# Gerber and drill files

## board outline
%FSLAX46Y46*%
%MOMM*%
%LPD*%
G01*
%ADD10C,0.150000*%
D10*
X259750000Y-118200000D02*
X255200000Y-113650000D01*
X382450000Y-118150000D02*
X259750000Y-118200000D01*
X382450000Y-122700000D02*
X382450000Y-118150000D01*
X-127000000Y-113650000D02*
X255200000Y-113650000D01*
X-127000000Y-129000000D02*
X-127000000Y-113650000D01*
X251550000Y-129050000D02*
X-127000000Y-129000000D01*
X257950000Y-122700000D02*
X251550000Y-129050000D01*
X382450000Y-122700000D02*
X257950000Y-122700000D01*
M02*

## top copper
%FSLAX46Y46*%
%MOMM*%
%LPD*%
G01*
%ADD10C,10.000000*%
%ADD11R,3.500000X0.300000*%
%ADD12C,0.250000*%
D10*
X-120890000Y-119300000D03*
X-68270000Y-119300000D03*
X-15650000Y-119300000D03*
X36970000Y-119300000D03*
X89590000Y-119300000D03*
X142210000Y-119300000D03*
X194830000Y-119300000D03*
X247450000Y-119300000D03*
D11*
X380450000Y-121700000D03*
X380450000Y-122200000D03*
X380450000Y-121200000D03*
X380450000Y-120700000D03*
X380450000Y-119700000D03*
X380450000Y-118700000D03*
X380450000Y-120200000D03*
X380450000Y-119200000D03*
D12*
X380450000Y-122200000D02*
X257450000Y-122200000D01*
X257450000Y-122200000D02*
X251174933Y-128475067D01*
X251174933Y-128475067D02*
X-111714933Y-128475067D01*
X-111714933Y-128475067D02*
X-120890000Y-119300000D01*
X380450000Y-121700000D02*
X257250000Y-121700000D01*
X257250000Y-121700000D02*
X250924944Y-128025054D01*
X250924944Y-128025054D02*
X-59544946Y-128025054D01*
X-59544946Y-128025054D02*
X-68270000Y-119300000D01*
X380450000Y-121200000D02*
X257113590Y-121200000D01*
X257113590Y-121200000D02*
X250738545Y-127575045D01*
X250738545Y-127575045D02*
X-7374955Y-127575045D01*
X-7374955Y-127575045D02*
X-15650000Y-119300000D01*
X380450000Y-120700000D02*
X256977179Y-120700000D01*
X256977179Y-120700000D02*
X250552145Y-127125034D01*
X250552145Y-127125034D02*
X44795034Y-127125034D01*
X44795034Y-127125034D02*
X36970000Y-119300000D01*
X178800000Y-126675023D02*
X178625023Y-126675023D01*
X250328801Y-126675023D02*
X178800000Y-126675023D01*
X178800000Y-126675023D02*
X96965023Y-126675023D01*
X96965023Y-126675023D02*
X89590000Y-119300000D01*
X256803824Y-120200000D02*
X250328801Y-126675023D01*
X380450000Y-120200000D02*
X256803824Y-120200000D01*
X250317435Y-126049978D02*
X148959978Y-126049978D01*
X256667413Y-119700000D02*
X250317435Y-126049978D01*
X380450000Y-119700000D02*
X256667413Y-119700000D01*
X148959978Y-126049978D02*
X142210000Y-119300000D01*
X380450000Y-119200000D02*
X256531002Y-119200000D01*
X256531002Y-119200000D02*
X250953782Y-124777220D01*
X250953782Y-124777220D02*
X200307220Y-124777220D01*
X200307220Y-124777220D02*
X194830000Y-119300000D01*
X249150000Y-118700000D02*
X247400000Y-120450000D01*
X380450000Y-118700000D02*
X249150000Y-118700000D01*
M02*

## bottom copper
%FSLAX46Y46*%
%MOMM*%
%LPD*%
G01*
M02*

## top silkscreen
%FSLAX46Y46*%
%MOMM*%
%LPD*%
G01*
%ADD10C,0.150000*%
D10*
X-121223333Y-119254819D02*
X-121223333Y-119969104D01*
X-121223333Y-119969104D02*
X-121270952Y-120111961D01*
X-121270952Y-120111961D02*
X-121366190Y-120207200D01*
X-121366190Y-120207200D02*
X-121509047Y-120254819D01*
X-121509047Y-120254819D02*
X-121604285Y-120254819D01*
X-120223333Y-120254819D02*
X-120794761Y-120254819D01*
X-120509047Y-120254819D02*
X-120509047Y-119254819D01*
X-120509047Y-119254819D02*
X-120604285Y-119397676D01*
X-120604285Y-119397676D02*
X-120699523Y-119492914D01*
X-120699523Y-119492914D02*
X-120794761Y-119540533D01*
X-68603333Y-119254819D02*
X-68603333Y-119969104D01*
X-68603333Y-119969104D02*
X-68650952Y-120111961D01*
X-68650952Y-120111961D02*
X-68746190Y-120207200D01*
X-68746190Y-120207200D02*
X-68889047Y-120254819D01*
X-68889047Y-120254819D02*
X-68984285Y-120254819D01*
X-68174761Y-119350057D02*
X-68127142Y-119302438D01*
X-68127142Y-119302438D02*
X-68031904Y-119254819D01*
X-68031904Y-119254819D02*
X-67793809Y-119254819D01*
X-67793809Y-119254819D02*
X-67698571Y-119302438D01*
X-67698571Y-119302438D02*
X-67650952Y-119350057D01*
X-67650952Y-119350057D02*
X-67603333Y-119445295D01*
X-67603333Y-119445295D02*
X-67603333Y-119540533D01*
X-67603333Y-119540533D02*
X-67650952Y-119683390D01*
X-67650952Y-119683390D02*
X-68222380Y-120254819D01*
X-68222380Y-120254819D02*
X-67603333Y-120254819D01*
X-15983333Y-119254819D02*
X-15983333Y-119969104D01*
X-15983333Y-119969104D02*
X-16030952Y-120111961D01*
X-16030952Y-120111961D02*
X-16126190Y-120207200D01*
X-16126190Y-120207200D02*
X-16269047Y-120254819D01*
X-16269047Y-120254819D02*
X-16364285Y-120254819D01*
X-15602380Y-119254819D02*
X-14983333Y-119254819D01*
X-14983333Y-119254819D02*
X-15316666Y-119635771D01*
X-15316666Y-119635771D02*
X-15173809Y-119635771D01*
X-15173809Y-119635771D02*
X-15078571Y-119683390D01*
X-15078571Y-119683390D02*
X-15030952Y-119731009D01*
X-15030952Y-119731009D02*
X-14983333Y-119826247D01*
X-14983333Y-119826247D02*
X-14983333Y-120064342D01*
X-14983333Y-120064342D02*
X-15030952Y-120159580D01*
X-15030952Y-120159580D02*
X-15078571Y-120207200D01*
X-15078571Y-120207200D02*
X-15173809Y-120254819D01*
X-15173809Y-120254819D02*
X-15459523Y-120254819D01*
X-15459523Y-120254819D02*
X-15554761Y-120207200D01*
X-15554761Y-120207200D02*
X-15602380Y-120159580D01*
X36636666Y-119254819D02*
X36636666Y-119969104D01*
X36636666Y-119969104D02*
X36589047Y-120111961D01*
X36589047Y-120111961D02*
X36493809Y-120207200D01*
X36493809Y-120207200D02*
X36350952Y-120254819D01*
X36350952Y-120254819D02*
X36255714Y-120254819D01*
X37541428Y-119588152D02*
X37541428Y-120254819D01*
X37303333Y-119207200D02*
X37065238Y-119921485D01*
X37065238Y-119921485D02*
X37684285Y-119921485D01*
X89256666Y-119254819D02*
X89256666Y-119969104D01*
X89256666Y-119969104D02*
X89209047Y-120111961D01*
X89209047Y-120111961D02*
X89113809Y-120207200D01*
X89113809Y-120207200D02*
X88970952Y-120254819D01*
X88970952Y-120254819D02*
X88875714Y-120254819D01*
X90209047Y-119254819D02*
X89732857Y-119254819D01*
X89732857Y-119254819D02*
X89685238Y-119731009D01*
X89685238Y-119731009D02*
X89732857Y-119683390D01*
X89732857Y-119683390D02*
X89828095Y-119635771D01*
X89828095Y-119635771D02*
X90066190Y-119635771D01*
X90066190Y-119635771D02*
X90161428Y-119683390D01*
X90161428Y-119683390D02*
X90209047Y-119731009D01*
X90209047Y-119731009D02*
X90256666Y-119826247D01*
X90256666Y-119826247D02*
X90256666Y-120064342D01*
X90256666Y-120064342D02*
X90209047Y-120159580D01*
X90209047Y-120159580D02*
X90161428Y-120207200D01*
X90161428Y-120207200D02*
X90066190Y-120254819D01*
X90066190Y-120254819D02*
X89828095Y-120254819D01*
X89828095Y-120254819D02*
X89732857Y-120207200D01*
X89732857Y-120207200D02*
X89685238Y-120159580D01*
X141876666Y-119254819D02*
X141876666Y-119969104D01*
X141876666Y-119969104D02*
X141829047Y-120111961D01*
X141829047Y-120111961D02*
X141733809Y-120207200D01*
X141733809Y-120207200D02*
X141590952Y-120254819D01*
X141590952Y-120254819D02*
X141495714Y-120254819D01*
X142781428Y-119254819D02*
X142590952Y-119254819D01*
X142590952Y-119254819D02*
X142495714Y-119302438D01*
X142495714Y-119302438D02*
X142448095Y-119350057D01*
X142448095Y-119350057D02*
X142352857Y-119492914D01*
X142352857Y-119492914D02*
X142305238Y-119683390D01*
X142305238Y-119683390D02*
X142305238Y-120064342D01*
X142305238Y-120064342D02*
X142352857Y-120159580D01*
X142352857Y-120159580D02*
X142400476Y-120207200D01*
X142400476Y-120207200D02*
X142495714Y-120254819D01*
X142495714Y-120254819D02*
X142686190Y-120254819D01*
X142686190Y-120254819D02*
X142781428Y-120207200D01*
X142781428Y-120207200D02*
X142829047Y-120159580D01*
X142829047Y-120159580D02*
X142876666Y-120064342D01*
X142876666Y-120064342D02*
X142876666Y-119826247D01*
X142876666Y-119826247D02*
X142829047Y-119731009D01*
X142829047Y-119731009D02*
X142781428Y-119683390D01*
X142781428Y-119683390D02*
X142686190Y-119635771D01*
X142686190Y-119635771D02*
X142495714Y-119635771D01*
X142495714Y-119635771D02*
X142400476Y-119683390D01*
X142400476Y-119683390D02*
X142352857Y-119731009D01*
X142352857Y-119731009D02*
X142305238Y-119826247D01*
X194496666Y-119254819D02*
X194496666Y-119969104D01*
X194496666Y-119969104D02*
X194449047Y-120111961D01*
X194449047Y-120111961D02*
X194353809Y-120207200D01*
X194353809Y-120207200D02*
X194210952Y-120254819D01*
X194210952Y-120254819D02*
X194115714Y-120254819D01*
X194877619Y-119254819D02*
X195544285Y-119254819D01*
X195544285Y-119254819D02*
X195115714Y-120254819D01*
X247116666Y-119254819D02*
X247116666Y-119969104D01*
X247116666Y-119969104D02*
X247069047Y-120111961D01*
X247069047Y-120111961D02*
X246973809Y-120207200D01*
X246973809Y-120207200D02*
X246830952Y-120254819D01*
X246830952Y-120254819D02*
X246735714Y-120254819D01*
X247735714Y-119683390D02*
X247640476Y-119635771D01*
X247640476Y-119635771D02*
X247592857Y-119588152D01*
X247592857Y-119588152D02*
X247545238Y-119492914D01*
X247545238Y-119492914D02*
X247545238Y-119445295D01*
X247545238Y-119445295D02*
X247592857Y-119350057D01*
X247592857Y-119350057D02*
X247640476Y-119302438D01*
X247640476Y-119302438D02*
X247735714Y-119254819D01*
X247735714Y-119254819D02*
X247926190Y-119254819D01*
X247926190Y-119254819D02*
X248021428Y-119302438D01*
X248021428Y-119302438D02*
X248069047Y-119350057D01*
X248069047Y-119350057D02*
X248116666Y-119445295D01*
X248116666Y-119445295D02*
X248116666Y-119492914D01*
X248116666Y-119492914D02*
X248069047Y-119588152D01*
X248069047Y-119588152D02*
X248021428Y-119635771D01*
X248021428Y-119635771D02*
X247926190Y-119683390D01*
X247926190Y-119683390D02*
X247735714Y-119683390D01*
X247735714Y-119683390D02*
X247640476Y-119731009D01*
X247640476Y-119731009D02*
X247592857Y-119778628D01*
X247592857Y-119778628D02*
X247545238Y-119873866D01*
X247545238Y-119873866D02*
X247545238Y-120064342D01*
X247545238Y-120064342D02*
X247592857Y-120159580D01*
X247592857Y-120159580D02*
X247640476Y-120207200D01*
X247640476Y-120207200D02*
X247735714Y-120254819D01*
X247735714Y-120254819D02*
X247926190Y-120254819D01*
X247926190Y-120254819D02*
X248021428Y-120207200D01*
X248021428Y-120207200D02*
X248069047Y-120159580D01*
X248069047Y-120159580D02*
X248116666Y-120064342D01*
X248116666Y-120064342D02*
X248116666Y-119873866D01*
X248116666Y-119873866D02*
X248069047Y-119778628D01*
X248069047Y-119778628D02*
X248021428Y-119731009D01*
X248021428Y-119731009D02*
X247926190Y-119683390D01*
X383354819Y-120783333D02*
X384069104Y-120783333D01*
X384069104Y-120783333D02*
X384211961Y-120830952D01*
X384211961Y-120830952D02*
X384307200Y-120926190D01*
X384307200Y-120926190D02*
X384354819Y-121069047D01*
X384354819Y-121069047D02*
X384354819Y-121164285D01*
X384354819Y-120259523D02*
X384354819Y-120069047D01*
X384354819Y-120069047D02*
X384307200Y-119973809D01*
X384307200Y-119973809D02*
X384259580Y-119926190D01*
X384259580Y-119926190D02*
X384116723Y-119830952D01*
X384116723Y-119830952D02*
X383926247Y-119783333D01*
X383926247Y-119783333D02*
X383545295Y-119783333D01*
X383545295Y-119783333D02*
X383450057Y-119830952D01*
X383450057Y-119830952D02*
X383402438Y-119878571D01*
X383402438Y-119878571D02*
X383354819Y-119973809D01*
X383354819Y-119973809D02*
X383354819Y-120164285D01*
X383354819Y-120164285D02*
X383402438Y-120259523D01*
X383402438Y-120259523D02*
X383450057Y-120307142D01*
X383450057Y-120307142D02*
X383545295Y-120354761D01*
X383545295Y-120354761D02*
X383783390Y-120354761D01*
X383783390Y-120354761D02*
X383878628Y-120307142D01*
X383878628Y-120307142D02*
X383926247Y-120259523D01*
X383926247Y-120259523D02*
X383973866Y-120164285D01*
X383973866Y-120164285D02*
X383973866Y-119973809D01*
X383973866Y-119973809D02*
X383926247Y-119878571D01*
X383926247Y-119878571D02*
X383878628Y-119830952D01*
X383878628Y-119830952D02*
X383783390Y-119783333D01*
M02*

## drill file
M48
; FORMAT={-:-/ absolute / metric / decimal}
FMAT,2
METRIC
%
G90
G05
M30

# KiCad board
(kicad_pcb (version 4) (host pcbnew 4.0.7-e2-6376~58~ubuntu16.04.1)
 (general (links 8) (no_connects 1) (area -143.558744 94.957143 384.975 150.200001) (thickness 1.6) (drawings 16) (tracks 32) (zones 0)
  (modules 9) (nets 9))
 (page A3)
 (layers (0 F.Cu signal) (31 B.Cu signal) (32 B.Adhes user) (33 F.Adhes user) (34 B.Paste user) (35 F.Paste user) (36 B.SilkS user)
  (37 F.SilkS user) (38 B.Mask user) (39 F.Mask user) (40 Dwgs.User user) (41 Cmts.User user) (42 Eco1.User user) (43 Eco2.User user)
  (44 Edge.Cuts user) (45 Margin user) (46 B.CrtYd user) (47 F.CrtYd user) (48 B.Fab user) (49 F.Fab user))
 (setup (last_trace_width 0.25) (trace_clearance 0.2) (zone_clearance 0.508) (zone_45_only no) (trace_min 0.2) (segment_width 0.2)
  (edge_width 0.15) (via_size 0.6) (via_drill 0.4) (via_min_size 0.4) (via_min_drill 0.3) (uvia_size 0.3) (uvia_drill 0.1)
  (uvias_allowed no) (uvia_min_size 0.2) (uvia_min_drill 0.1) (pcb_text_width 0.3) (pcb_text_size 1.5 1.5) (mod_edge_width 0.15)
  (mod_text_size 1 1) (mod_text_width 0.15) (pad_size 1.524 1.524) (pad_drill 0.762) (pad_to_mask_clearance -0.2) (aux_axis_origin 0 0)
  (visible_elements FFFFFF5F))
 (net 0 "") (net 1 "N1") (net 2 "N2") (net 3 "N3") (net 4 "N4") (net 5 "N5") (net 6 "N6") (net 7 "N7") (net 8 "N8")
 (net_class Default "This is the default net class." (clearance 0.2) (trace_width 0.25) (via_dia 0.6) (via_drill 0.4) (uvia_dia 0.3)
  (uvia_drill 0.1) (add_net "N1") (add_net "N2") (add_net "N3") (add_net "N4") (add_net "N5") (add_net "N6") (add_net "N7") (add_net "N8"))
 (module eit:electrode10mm (layer F.Cu) (at -120.89 119.3)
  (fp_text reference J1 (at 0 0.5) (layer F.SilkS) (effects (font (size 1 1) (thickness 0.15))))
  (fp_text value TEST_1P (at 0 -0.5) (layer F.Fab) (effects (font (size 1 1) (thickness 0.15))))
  (pad 1 smd circle (at 0 0) (size 10 10) (layers F.Cu F.Mask) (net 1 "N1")))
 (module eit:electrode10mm (layer F.Cu) (at -68.27 119.3)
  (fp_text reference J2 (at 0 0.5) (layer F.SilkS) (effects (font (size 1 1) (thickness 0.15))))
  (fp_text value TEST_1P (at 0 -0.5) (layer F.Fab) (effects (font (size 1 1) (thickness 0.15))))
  (pad 1 smd circle (at 0 0) (size 10 10) (layers F.Cu F.Mask) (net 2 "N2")))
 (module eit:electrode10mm (layer F.Cu) (at -15.65 119.3)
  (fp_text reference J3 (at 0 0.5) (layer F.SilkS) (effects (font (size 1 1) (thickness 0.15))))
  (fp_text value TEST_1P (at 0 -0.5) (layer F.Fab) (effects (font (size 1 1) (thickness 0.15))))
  (pad 1 smd circle (at 0 0) (size 10 10) (layers F.Cu F.Mask) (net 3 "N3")))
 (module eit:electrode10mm (layer F.Cu) (at 36.97 119.3)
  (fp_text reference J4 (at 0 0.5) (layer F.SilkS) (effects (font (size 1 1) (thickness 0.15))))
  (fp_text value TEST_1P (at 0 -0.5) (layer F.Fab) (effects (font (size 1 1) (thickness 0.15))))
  (pad 1 smd circle (at 0 0) (size 10 10) (layers F.Cu F.Mask) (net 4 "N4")))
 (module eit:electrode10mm (layer F.Cu) (at 89.59 119.3)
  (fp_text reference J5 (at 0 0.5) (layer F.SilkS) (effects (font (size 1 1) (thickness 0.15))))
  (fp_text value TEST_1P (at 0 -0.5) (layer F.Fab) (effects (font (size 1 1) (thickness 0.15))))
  (pad 1 smd circle (at 0 0) (size 10 10) (layers F.Cu F.Mask) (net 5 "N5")))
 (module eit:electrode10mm (layer F.Cu) (at 142.21 119.3)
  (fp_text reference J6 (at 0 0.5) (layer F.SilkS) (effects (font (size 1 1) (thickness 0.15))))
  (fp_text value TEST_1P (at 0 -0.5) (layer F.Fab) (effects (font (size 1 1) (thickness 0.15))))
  (pad 1 smd circle (at 0 0) (size 10 10) (layers F.Cu F.Mask) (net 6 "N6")))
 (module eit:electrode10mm (layer F.Cu) (at 194.83 119.3)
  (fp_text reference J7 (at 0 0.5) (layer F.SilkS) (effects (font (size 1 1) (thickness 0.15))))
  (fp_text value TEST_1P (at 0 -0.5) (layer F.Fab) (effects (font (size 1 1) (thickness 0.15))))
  (pad 1 smd circle (at 0 0) (size 10 10) (layers F.Cu F.Mask) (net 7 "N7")))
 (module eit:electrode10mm (layer F.Cu) (at 247.45 119.3)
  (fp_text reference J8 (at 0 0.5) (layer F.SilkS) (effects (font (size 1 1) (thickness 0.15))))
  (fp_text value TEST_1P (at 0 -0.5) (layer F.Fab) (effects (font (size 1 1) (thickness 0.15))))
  (pad 1 smd circle (at 0 0) (size 10 10) (layers F.Cu F.Mask) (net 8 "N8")))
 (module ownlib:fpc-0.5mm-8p (layer F.Cu) (at 383.4 120.45 90)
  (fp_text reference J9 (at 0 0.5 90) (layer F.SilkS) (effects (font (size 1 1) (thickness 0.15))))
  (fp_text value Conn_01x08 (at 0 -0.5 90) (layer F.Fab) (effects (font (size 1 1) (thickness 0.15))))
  (pad 2 smd rect (at -1.25 -2.95 90) (size 0.3 3.5) (layers F.Cu F.Paste F.Mask) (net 2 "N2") (solder_mask_margin 0.2))
  (pad 1 smd rect (at -1.75 -2.95 90) (size 0.3 3.5) (layers F.Cu F.Paste F.Mask) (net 1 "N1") (solder_mask_margin 0.2))
  (pad 3 smd rect (at -0.75 -2.95 90) (size 0.3 3.5) (layers F.Cu F.Paste F.Mask) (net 3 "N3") (solder_mask_margin 0.2))
  (pad 4 smd rect (at -0.25 -2.95 90) (size 0.3 3.5) (layers F.Cu F.Paste F.Mask) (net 4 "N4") (solder_mask_margin 0.2))
  (pad 6 smd rect (at 0.75 -2.95 90) (size 0.3 3.5) (layers F.Cu F.Paste F.Mask) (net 6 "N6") (solder_mask_margin 0.2))
  (pad 8 smd rect (at 1.75 -2.95 90) (size 0.3 3.5) (layers F.Cu F.Paste F.Mask) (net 8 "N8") (solder_mask_margin 0.2))
  (pad 5 smd rect (at 0.25 -2.95 90) (size 0.3 3.5) (layers F.Cu F.Paste F.Mask) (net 5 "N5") (solder_mask_margin 0.2))
  (pad 7 smd rect (at 1.25 -2.95 90) (size 0.3 3.5) (layers F.Cu F.Paste F.Mask) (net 7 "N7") (solder_mask_margin 0.2)))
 (gr_line (start 259.75 118.2) (end 255.2 113.65) (layer Edge.Cuts) (width 0.15))
 (gr_line (start 382.45 118.15) (end 259.75 118.2) (layer Edge.Cuts) (width 0.15))
 (gr_line (start 382.45 122.7) (end 382.45 118.15) (layer Edge.Cuts) (width 0.15))
 (gr_line (start -127 113.65) (end 255.2 113.65) (layer Edge.Cuts) (width 0.15))
 (gr_line (start -127 129) (end -127 113.65) (layer Edge.Cuts) (width 0.15))
 (gr_line (start 251.55 129.05) (end -127 129) (layer Edge.Cuts) (width 0.15))
 (gr_line (start 257.95 122.7) (end 251.55 129.05) (layer Edge.Cuts) (width 0.15))
 (gr_line (start 382.45 122.7) (end 257.95 122.7) (layer Edge.Cuts) (width 0.15))
 (segment (start 380.45 122.2) (end 257.45 122.2) (width 0.25) (layer F.Cu) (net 1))
 (segment (start 257.45 122.2) (end 251.174933 128.475067) (width 0.25) (layer F.Cu) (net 1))
 (segment (start 251.174933 128.475067) (end -111.714933 128.475067) (width 0.25) (layer F.Cu) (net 1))
 (segment (start -111.714933 128.475067) (end -120.89 119.3) (width 0.25) (layer F.Cu) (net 1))
 (segment (start 380.45 121.7) (end 257.25 121.7) (width 0.25) (layer F.Cu) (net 2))
 (segment (start 257.25 121.7) (end 250.924944 128.025054) (width 0.25) (layer F.Cu) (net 2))
 (segment (start 250.924944 128.025054) (end -59.544946 128.025054) (width 0.25) (layer F.Cu) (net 2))
 (segment (start -59.544946 128.025054) (end -68.27 119.3) (width 0.25) (layer F.Cu) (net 2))
 (segment (start 380.45 121.2) (end 257.11359 121.2) (width 0.25) (layer F.Cu) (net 3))
 (segment (start 257.11359 121.2) (end 250.738545 127.575045) (width 0.25) (layer F.Cu) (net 3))
 (segment (start 250.738545 127.575045) (end -7.374955 127.575045) (width 0.25) (layer F.Cu) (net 3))
 (segment (start -7.374955 127.575045) (end -15.65 119.3) (width 0.25) (layer F.Cu) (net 3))
 (segment (start 380.45 120.7) (end 256.977179 120.7) (width 0.25) (layer F.Cu) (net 4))
 (segment (start 256.977179 120.7) (end 250.552145 127.125034) (width 0.25) (layer F.Cu) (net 4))
 (segment (start 250.552145 127.125034) (end 44.795034 127.125034) (width 0.25) (layer F.Cu) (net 4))
 (segment (start 44.795034 127.125034) (end 36.97 119.3) (width 0.25) (layer F.Cu) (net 4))
 (segment (start 178.8 126.675023) (end 178.625023 126.675023) (width 0.25) (layer F.Cu) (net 5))
 (segment (start 250.328801 126.675023) (end 178.8 126.675023) (width 0.25) (layer F.Cu) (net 5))
 (segment (start 178.8 126.675023) (end 96.965023 126.675023) (width 0.25) (layer F.Cu) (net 5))
 (segment (start 96.965023 126.675023) (end 89.59 119.3) (width 0.25) (layer F.Cu) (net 5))
 (segment (start 256.803824 120.2) (end 250.328801 126.675023) (width 0.25) (layer F.Cu) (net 5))
 (segment (start 380.45 120.2) (end 256.803824 120.2) (width 0.25) (layer F.Cu) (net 5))
 (segment (start 250.317435 126.049978) (end 148.959978 126.049978) (width 0.25) (layer F.Cu) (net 6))
 (segment (start 256.667413 119.7) (end 250.317435 126.049978) (width 0.25) (layer F.Cu) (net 6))
 (segment (start 380.45 119.7) (end 256.667413 119.7) (width 0.25) (layer F.Cu) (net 6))
 (segment (start 148.959978 126.049978) (end 142.21 119.3) (width 0.25) (layer F.Cu) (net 6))
 (segment (start 380.45 119.2) (end 256.531002 119.2) (width 0.25) (layer F.Cu) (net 7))
 (segment (start 256.531002 119.2) (end 250.953782 124.77722) (width 0.25) (layer F.Cu) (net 7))
 (segment (start 250.953782 124.77722) (end 200.30722 124.77722) (width 0.25) (layer F.Cu) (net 7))
 (segment (start 200.30722 124.77722) (end 194.83 119.3) (width 0.25) (layer F.Cu) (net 7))
 (segment (start 249.15 118.7) (end 247.4 120.45) (width 0.25) (layer F.Cu) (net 8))
 (segment (start 380.45 118.7) (end 249.15 118.7) (width 0.25) (layer F.Cu) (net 8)))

